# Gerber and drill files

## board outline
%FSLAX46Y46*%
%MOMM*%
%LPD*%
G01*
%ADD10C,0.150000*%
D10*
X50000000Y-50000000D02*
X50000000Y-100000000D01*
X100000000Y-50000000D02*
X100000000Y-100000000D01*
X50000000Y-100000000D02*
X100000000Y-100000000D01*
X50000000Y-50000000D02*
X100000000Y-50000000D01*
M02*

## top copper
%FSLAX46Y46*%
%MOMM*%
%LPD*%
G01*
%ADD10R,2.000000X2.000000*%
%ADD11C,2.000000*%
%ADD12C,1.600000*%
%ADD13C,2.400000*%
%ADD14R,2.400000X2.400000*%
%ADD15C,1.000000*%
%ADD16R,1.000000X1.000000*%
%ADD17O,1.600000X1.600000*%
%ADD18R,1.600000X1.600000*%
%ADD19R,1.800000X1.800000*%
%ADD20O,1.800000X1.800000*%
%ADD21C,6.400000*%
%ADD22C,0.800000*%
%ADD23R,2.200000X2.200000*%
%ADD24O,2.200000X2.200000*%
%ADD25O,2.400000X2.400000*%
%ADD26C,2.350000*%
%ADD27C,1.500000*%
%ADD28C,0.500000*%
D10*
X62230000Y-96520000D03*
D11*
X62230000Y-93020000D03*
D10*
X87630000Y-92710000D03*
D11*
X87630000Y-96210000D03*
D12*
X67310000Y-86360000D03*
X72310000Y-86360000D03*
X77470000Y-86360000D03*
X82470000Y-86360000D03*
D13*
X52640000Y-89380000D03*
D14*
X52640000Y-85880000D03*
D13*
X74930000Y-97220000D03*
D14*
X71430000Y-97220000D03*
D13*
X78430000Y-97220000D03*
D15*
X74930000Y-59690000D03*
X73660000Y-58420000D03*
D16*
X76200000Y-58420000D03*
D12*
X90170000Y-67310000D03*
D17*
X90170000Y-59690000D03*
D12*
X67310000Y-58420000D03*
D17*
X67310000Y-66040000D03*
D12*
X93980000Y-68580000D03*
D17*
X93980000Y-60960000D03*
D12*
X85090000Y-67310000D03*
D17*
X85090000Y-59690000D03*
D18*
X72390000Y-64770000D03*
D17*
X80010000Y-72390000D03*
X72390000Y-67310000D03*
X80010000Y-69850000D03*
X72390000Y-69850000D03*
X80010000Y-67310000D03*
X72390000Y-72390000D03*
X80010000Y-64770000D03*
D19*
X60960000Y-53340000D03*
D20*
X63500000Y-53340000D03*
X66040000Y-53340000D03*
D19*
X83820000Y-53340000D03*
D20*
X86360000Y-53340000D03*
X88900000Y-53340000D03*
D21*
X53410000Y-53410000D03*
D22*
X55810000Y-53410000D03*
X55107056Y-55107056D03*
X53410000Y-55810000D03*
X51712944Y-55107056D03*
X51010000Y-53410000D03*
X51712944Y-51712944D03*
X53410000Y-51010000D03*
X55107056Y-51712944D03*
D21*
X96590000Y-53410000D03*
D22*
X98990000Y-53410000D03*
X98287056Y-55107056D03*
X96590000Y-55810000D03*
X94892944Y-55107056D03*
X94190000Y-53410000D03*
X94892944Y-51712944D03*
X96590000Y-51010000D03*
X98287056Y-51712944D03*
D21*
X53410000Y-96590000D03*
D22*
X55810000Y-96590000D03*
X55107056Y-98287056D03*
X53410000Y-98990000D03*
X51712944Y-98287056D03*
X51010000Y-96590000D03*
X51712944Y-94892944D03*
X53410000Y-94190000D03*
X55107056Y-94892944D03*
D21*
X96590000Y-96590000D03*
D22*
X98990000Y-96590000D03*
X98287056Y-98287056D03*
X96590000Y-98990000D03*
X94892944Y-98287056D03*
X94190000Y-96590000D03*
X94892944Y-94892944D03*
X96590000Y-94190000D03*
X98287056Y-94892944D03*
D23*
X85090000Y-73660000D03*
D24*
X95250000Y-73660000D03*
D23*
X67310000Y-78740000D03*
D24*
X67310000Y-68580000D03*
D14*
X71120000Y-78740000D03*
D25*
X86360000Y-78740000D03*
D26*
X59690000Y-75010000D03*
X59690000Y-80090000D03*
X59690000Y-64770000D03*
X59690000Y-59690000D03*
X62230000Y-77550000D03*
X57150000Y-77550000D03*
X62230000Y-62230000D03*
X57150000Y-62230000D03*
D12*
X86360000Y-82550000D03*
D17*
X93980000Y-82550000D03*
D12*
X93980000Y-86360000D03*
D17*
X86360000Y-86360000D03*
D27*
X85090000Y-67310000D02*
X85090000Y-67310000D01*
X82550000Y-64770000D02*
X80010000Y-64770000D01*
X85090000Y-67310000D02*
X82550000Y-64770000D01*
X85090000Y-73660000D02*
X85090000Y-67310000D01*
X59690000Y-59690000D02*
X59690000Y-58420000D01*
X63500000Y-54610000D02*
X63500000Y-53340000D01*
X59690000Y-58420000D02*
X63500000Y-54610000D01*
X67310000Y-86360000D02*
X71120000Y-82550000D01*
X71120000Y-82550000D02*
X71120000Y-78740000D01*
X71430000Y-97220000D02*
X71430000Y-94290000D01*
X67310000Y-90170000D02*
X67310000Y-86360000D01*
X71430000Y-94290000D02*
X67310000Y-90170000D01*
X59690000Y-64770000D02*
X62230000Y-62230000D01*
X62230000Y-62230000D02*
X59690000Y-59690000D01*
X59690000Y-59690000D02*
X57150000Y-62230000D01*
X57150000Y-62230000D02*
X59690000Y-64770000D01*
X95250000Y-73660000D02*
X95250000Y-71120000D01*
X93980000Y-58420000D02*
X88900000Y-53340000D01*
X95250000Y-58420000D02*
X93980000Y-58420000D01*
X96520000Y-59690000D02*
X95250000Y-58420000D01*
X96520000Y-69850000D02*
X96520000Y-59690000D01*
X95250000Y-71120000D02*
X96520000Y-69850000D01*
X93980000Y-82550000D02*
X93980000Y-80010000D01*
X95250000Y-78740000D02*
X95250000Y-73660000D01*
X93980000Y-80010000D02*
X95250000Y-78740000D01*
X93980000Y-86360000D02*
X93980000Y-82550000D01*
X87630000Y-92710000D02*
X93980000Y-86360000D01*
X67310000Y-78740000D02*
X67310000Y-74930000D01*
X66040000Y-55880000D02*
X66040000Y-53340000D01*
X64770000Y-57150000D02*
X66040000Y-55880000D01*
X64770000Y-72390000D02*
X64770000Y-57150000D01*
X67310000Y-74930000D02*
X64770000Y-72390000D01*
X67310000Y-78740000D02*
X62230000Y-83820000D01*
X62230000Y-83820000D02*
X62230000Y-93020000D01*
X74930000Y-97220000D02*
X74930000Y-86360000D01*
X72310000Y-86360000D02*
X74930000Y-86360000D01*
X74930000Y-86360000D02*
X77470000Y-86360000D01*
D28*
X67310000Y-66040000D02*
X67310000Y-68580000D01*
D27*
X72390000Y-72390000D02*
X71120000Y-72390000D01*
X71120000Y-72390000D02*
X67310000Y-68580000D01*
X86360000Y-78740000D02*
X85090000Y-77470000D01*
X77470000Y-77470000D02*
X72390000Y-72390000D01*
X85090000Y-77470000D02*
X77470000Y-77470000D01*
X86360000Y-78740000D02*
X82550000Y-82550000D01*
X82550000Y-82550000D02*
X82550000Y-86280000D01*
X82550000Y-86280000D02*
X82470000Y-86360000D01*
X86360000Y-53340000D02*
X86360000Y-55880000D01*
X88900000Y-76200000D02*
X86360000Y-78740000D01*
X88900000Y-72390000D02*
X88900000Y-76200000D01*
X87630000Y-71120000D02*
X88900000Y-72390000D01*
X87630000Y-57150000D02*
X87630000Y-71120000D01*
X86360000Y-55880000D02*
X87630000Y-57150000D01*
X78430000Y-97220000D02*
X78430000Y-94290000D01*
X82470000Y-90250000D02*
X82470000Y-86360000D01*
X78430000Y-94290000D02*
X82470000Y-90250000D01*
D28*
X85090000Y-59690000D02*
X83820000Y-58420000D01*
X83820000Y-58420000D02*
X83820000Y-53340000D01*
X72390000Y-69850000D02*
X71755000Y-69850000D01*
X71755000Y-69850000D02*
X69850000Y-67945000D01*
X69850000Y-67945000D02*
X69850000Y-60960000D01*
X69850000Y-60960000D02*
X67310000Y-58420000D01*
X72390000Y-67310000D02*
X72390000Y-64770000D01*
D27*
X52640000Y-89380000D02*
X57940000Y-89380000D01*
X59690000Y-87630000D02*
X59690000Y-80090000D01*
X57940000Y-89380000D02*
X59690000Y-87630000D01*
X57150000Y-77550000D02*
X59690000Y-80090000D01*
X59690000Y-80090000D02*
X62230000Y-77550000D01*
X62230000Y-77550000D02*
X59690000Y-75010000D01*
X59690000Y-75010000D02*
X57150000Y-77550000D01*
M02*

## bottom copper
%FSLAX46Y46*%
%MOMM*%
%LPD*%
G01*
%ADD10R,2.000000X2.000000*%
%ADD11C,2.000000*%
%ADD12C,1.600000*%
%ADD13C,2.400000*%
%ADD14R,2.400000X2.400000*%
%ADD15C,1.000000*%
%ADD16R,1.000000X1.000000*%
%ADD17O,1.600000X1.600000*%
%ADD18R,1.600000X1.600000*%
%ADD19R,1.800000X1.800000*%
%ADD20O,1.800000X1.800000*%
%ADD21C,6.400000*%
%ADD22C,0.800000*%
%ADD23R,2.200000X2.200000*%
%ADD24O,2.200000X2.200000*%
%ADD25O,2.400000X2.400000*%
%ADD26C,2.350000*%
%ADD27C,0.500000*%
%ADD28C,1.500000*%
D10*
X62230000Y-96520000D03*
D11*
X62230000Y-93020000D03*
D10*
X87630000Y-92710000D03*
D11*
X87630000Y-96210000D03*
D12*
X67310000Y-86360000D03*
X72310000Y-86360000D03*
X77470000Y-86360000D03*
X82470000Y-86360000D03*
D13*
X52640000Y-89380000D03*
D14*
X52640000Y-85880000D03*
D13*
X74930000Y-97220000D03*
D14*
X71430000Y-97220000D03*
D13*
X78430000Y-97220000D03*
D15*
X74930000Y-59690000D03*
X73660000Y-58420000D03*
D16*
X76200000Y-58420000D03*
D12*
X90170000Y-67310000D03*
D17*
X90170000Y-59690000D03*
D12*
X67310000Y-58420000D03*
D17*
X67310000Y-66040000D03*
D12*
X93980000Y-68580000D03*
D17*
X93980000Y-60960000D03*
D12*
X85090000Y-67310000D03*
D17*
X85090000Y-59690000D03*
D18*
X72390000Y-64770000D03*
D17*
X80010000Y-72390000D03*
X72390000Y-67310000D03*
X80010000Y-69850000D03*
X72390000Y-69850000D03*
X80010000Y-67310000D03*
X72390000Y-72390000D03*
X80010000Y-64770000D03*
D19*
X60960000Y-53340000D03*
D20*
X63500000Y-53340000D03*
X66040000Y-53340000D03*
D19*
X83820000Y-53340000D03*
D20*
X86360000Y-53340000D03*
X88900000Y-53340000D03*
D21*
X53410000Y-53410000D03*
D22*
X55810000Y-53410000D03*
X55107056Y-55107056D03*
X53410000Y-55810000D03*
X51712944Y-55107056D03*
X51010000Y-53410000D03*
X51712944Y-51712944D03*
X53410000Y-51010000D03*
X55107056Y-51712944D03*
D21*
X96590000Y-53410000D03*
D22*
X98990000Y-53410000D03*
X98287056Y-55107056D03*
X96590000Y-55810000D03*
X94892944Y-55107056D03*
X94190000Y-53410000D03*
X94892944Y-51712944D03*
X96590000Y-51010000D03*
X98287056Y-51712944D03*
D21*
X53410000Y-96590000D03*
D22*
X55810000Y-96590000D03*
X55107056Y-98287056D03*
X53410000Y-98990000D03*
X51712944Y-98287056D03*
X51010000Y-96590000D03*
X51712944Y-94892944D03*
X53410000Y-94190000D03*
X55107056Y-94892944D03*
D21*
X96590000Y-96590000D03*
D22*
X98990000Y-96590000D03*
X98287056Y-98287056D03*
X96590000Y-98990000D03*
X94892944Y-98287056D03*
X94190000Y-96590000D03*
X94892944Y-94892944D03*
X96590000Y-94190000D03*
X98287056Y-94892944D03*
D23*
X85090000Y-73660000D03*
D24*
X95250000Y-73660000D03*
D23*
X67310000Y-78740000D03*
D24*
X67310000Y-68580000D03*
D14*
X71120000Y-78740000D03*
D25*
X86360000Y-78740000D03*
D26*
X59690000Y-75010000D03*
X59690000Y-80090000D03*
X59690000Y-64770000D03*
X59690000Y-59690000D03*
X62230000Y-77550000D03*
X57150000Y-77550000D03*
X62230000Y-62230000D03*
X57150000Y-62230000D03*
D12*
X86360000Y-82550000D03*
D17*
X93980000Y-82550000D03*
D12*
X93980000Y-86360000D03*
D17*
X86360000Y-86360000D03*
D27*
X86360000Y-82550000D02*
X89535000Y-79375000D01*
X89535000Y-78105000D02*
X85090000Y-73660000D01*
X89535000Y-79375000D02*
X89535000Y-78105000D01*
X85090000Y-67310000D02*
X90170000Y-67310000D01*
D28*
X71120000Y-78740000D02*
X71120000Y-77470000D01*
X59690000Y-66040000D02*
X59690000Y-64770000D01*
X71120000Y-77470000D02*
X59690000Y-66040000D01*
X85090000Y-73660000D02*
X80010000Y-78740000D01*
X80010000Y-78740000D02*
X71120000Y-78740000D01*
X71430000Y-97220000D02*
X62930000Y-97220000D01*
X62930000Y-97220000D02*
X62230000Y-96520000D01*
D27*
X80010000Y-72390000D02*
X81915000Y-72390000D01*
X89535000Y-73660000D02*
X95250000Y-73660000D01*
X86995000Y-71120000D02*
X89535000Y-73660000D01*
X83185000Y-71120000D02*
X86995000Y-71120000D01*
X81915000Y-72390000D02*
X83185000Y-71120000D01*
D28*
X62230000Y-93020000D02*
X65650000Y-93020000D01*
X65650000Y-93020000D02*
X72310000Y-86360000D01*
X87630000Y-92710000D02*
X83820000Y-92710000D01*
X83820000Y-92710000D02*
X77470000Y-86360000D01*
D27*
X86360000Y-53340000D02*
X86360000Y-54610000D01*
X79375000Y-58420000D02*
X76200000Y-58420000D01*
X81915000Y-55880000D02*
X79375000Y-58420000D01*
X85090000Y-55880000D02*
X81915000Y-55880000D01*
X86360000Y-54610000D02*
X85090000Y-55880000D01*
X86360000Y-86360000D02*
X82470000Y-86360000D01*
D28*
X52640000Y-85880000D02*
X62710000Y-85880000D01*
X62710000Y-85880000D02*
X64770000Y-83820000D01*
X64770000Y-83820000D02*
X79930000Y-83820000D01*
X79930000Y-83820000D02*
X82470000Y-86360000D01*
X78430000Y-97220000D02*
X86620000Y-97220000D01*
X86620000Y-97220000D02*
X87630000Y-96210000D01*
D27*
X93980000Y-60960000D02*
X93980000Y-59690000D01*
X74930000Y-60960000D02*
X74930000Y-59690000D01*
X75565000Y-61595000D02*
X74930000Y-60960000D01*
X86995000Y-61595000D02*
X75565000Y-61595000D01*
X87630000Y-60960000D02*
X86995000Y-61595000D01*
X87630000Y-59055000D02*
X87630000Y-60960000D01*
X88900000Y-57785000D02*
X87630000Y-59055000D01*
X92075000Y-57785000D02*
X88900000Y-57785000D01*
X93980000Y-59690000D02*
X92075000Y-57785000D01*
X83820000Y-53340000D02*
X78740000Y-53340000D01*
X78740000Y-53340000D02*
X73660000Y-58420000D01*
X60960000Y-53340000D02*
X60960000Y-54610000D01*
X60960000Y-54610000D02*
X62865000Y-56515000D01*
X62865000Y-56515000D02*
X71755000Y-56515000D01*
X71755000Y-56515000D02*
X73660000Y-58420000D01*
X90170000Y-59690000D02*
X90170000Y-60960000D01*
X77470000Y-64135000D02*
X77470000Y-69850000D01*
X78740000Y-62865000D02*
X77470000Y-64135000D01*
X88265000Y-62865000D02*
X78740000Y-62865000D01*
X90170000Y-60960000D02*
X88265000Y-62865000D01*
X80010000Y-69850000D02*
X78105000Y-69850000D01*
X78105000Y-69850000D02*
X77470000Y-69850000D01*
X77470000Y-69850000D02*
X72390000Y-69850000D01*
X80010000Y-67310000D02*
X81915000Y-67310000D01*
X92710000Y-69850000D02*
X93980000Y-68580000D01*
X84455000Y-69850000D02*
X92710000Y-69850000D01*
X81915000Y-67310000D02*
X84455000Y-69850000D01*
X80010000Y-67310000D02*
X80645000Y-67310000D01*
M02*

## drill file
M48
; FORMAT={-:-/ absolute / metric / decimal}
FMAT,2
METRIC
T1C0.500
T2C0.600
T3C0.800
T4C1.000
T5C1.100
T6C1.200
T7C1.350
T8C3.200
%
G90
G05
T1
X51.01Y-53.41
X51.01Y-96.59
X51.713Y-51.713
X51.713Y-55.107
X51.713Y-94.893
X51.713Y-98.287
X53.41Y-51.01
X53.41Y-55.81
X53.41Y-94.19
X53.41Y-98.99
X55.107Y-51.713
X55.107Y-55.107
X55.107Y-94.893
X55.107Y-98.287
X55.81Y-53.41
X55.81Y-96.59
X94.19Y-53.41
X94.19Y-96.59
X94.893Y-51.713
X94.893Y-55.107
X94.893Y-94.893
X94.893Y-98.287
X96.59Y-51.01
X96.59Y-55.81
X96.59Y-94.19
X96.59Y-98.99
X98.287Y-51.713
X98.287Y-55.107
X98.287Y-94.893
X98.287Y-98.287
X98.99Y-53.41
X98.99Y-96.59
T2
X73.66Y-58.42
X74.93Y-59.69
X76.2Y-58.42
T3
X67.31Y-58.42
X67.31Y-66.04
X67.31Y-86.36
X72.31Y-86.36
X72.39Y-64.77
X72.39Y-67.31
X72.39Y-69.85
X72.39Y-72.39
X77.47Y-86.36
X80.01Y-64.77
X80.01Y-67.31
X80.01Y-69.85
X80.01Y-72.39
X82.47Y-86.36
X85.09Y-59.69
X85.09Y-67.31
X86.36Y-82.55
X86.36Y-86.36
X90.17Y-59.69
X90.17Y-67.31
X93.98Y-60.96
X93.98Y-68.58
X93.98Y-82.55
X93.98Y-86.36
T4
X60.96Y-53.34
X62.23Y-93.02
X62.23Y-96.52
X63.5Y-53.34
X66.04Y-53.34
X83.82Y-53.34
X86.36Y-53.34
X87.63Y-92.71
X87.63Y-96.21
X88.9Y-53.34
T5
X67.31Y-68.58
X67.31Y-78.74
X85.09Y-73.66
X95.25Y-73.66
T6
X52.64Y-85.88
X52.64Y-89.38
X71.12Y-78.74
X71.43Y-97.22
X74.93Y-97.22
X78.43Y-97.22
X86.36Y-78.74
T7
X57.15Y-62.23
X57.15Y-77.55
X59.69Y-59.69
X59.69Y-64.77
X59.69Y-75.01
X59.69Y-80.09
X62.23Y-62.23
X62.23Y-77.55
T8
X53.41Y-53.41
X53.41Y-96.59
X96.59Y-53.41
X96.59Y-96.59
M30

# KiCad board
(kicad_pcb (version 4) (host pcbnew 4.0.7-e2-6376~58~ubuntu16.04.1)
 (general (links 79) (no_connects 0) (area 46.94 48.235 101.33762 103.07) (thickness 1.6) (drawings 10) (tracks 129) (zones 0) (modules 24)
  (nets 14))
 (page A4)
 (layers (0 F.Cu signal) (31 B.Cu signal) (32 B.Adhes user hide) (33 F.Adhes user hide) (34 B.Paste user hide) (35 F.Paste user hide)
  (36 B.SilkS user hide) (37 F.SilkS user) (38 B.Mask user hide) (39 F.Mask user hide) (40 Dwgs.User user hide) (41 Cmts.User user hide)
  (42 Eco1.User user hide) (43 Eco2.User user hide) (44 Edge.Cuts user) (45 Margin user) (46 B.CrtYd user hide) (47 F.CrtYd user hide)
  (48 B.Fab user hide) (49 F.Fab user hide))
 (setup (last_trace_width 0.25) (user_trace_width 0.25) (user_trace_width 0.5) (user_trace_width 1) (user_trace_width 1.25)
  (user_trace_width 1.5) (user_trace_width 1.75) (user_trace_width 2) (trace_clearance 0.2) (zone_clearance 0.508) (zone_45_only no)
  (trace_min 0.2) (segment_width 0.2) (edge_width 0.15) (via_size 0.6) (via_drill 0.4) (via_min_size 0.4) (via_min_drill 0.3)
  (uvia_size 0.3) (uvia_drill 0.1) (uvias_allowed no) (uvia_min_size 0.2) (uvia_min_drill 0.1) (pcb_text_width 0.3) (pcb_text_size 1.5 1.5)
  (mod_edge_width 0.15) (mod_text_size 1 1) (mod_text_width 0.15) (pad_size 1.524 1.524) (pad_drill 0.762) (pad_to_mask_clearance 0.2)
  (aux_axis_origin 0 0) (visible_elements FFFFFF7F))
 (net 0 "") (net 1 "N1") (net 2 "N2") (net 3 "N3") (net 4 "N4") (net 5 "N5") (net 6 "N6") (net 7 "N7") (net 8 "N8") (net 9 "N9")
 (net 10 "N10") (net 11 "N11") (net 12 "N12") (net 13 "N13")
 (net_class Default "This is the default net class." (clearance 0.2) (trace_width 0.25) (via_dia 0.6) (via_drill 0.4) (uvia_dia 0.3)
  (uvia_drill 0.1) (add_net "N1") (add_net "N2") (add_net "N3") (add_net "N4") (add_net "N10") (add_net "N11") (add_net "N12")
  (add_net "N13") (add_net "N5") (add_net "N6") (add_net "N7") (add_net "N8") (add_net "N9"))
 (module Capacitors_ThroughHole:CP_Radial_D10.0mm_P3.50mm (layer F.Cu) (at 62.23 96.52 90)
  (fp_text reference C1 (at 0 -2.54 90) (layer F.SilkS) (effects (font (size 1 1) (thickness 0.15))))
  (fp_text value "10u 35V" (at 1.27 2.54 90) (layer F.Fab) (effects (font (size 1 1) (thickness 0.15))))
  (pad 1 thru_hole rect (at 0 0 90) (size 2 2) (drill 1) (layers *.Cu *.Mask) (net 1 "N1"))
  (pad 2 thru_hole circle (at 3.5 0 90) (size 2 2) (drill 1) (layers *.Cu *.Mask) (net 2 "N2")))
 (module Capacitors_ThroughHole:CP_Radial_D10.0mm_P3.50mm (layer F.Cu) (at 87.63 92.71 270)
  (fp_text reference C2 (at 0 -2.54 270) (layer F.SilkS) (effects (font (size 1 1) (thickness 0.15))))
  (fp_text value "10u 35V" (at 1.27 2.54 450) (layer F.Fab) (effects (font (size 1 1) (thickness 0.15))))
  (pad 1 thru_hole rect (at 0 0 270) (size 2 2) (drill 1) (layers *.Cu *.Mask) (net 2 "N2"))
  (pad 2 thru_hole circle (at 3.5 0 270) (size 2 2) (drill 1) (layers *.Cu *.Mask) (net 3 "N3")))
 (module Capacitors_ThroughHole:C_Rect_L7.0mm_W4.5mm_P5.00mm (layer F.Cu) (at 67.31 86.36)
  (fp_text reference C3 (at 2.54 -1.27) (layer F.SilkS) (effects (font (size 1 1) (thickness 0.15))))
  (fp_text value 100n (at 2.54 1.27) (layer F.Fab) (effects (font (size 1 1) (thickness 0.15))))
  (pad 1 thru_hole circle (at 0 0) (size 1.6 1.6) (drill 0.8) (layers *.Cu *.Mask) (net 1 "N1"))
  (pad 2 thru_hole circle (at 5 0) (size 1.6 1.6) (drill 0.8) (layers *.Cu *.Mask) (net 2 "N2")))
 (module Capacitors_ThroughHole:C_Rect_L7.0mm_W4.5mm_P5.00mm (layer F.Cu) (at 77.47 86.36)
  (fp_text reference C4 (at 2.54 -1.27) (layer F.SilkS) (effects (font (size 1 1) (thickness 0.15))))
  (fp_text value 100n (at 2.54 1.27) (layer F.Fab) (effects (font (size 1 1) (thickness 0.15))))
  (pad 1 thru_hole circle (at 0 0) (size 1.6 1.6) (drill 0.8) (layers *.Cu *.Mask) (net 2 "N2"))
  (pad 2 thru_hole circle (at 5 0) (size 1.6 1.6) (drill 0.8) (layers *.Cu *.Mask) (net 3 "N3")))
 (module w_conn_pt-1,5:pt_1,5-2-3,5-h (layer F.Cu) (at 53.34 87.63 90)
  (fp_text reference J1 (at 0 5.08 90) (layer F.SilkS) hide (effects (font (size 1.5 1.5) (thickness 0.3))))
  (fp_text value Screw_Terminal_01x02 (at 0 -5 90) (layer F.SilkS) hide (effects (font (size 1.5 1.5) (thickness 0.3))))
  (pad 2 thru_hole circle (at -1.75 -0.7 90) (size 2.4 2.4) (drill 1.2) (layers *.Cu *.Mask F.SilkS) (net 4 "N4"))
  (pad 1 thru_hole rect (at 1.75 -0.7 90) (size 2.4 2.4) (drill 1.2) (layers *.Cu *.Mask F.SilkS) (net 3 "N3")))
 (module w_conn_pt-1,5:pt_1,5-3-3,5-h (layer F.Cu) (at 74.93 96.52 180)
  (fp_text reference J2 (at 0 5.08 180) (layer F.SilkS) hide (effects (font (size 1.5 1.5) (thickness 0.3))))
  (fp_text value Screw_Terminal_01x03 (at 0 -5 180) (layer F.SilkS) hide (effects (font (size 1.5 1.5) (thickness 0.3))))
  (pad 2 thru_hole circle (at 0 -0.7 180) (size 2.4 2.4) (drill 1.2) (layers *.Cu *.Mask F.SilkS) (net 2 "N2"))
  (pad 1 thru_hole rect (at 3.5 -0.7 180) (size 2.4 2.4) (drill 1.2) (layers *.Cu *.Mask F.SilkS) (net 1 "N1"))
  (pad 3 thru_hole circle (at -3.5 -0.7 180) (size 2.4 2.4) (drill 1.2) (layers *.Cu *.Mask F.SilkS) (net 3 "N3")))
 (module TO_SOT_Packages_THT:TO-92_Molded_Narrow (layer F.Cu) (at 76.2 58.42 180)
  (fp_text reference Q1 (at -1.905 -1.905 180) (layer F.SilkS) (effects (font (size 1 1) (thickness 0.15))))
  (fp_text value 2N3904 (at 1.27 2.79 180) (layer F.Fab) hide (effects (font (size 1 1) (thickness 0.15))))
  (pad 2 thru_hole circle (at 1.27 -1.27 270) (size 1 1) (drill 0.6) (layers *.Cu *.Mask) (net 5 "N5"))
  (pad 3 thru_hole circle (at 2.54 0 270) (size 1 1) (drill 0.6) (layers *.Cu *.Mask) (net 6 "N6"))
  (pad 1 thru_hole rect (at 0 0 270) (size 1 1) (drill 0.6) (layers *.Cu *.Mask) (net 3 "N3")))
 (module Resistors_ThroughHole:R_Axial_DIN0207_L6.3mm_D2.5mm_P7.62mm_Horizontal (layer F.Cu) (at 90.17 67.31 90)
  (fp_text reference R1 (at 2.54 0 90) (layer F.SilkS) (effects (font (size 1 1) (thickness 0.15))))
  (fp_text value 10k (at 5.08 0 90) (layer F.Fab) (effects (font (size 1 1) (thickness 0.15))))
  (pad 1 thru_hole circle (at 0 0 90) (size 1.6 1.6) (drill 0.8) (layers *.Cu *.Mask) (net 1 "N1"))
  (pad 2 thru_hole oval (at 7.62 0 90) (size 1.6 1.6) (drill 0.8) (layers *.Cu *.Mask) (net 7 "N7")))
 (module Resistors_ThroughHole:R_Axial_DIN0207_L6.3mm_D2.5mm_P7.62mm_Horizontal (layer F.Cu) (at 67.31 58.42 270)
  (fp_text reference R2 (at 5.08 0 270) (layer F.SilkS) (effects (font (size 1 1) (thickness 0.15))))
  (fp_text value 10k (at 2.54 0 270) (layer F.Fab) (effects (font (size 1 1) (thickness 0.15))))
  (pad 1 thru_hole circle (at 0 0 270) (size 1.6 1.6) (drill 0.8) (layers *.Cu *.Mask) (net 7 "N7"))
  (pad 2 thru_hole oval (at 7.62 0 270) (size 1.6 1.6) (drill 0.8) (layers *.Cu *.Mask) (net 3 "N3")))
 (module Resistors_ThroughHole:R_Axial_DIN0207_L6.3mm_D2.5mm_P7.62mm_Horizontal (layer F.Cu) (at 93.98 68.58 90)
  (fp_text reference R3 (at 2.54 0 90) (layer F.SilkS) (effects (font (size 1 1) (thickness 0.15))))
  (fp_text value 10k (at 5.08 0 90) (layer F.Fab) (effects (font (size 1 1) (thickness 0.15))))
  (pad 1 thru_hole circle (at 0 0 90) (size 1.6 1.6) (drill 0.8) (layers *.Cu *.Mask) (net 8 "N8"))
  (pad 2 thru_hole oval (at 7.62 0 90) (size 1.6 1.6) (drill 0.8) (layers *.Cu *.Mask) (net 5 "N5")))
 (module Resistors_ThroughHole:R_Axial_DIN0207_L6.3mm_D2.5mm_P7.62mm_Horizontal (layer F.Cu) (at 85.09 67.31 90)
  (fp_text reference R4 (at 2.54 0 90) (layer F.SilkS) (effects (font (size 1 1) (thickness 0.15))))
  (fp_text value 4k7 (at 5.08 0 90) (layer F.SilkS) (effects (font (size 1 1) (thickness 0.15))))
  (pad 1 thru_hole circle (at 0 0 90) (size 1.6 1.6) (drill 0.8) (layers *.Cu *.Mask) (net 1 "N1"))
  (pad 2 thru_hole oval (at 7.62 0 90) (size 1.6 1.6) (drill 0.8) (layers *.Cu *.Mask) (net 6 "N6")))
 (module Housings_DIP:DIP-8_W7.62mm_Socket (layer F.Cu) (at 72.39 64.77)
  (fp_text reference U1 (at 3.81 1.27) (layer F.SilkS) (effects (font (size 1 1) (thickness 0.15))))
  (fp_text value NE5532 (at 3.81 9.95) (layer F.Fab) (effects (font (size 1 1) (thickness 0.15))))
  (pad 1 thru_hole rect (at 0 0) (size 1.6 1.6) (drill 0.8) (layers *.Cu *.Mask) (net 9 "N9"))
  (pad 5 thru_hole oval (at 7.62 7.62) (size 1.6 1.6) (drill 0.8) (layers *.Cu *.Mask) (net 2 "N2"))
  (pad 2 thru_hole oval (at 0 2.54) (size 1.6 1.6) (drill 0.8) (layers *.Cu *.Mask) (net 9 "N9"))
  (pad 6 thru_hole oval (at 7.62 5.08) (size 1.6 1.6) (drill 0.8) (layers *.Cu *.Mask) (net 7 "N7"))
  (pad 3 thru_hole oval (at 0 5.08) (size 1.6 1.6) (drill 0.8) (layers *.Cu *.Mask) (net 7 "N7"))
  (pad 7 thru_hole oval (at 7.62 2.54) (size 1.6 1.6) (drill 0.8) (layers *.Cu *.Mask) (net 8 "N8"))
  (pad 4 thru_hole oval (at 0 7.62) (size 1.6 1.6) (drill 0.8) (layers *.Cu *.Mask) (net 3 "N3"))
  (pad 8 thru_hole oval (at 7.62 0) (size 1.6 1.6) (drill 0.8) (layers *.Cu *.Mask) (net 1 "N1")))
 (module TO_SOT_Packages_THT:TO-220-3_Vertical (layer F.Cu) (at 60.96 53.34)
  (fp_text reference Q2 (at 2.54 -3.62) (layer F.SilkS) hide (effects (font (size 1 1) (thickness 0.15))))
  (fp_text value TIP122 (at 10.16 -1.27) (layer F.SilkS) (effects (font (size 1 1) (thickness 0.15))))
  (pad 1 thru_hole rect (at 0 0) (size 1.8 1.8) (drill 1) (layers *.Cu *.Mask) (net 6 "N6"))
  (pad 2 thru_hole oval (at 2.54 0) (size 1.8 1.8) (drill 1) (layers *.Cu *.Mask) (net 1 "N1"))
  (pad 3 thru_hole oval (at 5.08 0) (size 1.8 1.8) (drill 1) (layers *.Cu *.Mask) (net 2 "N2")))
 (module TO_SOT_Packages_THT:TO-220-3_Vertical (layer F.Cu) (at 83.82 53.34)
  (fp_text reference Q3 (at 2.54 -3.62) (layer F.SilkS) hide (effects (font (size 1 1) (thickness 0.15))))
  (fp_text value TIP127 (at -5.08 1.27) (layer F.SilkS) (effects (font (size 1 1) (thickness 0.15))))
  (pad 1 thru_hole rect (at 0 0) (size 1.8 1.8) (drill 1) (layers *.Cu *.Mask) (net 6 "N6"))
  (pad 2 thru_hole oval (at 2.54 0) (size 1.8 1.8) (drill 1) (layers *.Cu *.Mask) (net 3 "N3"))
  (pad 3 thru_hole oval (at 5.08 0) (size 1.8 1.8) (drill 1) (layers *.Cu *.Mask) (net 2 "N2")))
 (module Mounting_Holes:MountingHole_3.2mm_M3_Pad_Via (layer F.Cu) (at 53.41 53.41)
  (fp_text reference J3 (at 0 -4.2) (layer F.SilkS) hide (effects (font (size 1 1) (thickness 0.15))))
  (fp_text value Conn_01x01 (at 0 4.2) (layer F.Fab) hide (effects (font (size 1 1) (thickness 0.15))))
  (pad 1 thru_hole circle (at 0 0) (size 6.4 6.4) (drill 3.2) (layers *.Cu *.Mask) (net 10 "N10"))
  (pad 1 thru_hole circle (at 2.4 0) (size 0.8 0.8) (drill 0.5) (layers *.Cu *.Mask) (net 10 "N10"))
  (pad 1 thru_hole circle (at 1.697056 1.697056) (size 0.8 0.8) (drill 0.5) (layers *.Cu *.Mask) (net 10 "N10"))
  (pad 1 thru_hole circle (at 0 2.4) (size 0.8 0.8) (drill 0.5) (layers *.Cu *.Mask) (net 10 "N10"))
  (pad 1 thru_hole circle (at -1.697056 1.697056) (size 0.8 0.8) (drill 0.5) (layers *.Cu *.Mask) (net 10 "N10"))
  (pad 1 thru_hole circle (at -2.4 0) (size 0.8 0.8) (drill 0.5) (layers *.Cu *.Mask) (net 10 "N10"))
  (pad 1 thru_hole circle (at -1.697056 -1.697056) (size 0.8 0.8) (drill 0.5) (layers *.Cu *.Mask) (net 10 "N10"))
  (pad 1 thru_hole circle (at 0 -2.4) (size 0.8 0.8) (drill 0.5) (layers *.Cu *.Mask) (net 10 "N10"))
  (pad 1 thru_hole circle (at 1.697056 -1.697056) (size 0.8 0.8) (drill 0.5) (layers *.Cu *.Mask) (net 10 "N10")))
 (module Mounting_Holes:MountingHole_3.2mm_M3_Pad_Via (layer F.Cu) (at 96.59 53.41)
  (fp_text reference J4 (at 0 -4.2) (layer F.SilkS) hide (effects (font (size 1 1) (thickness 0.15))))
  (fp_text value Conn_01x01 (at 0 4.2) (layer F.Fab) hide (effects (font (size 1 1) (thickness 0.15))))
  (pad 1 thru_hole circle (at 0 0) (size 6.4 6.4) (drill 3.2) (layers *.Cu *.Mask) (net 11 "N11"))
  (pad 1 thru_hole circle (at 2.4 0) (size 0.8 0.8) (drill 0.5) (layers *.Cu *.Mask) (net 11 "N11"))
  (pad 1 thru_hole circle (at 1.697056 1.697056) (size 0.8 0.8) (drill 0.5) (layers *.Cu *.Mask) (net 11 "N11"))
  (pad 1 thru_hole circle (at 0 2.4) (size 0.8 0.8) (drill 0.5) (layers *.Cu *.Mask) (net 11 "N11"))
  (pad 1 thru_hole circle (at -1.697056 1.697056) (size 0.8 0.8) (drill 0.5) (layers *.Cu *.Mask) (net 11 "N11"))
  (pad 1 thru_hole circle (at -2.4 0) (size 0.8 0.8) (drill 0.5) (layers *.Cu *.Mask) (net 11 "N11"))
  (pad 1 thru_hole circle (at -1.697056 -1.697056) (size 0.8 0.8) (drill 0.5) (layers *.Cu *.Mask) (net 11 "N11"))
  (pad 1 thru_hole circle (at 0 -2.4) (size 0.8 0.8) (drill 0.5) (layers *.Cu *.Mask) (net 11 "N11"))
  (pad 1 thru_hole circle (at 1.697056 -1.697056) (size 0.8 0.8) (drill 0.5) (layers *.Cu *.Mask) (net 11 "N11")))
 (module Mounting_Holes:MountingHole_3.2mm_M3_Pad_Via (layer F.Cu) (at 53.41 96.59)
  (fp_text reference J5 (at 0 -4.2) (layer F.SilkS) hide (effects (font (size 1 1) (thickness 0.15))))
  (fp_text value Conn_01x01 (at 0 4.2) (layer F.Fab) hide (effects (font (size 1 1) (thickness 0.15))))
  (pad 1 thru_hole circle (at 0 0) (size 6.4 6.4) (drill 3.2) (layers *.Cu *.Mask) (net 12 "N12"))
  (pad 1 thru_hole circle (at 2.4 0) (size 0.8 0.8) (drill 0.5) (layers *.Cu *.Mask) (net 12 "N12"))
  (pad 1 thru_hole circle (at 1.697056 1.697056) (size 0.8 0.8) (drill 0.5) (layers *.Cu *.Mask) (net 12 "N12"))
  (pad 1 thru_hole circle (at 0 2.4) (size 0.8 0.8) (drill 0.5) (layers *.Cu *.Mask) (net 12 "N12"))
  (pad 1 thru_hole circle (at -1.697056 1.697056) (size 0.8 0.8) (drill 0.5) (layers *.Cu *.Mask) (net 12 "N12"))
  (pad 1 thru_hole circle (at -2.4 0) (size 0.8 0.8) (drill 0.5) (layers *.Cu *.Mask) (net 12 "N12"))
  (pad 1 thru_hole circle (at -1.697056 -1.697056) (size 0.8 0.8) (drill 0.5) (layers *.Cu *.Mask) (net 12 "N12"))
  (pad 1 thru_hole circle (at 0 -2.4) (size 0.8 0.8) (drill 0.5) (layers *.Cu *.Mask) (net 12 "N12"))
  (pad 1 thru_hole circle (at 1.697056 -1.697056) (size 0.8 0.8) (drill 0.5) (layers *.Cu *.Mask) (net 12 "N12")))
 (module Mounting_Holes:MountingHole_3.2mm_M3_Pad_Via (layer F.Cu) (at 96.59 96.59)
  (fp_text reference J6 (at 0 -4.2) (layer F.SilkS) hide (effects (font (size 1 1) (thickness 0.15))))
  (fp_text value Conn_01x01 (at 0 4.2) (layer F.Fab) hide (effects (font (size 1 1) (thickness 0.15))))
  (pad 1 thru_hole circle (at 0 0) (size 6.4 6.4) (drill 3.2) (layers *.Cu *.Mask) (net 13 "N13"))
  (pad 1 thru_hole circle (at 2.4 0) (size 0.8 0.8) (drill 0.5) (layers *.Cu *.Mask) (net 13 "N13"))
  (pad 1 thru_hole circle (at 1.697056 1.697056) (size 0.8 0.8) (drill 0.5) (layers *.Cu *.Mask) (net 13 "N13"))
  (pad 1 thru_hole circle (at 0 2.4) (size 0.8 0.8) (drill 0.5) (layers *.Cu *.Mask) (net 13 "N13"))
  (pad 1 thru_hole circle (at -1.697056 1.697056) (size 0.8 0.8) (drill 0.5) (layers *.Cu *.Mask) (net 13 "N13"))
  (pad 1 thru_hole circle (at -2.4 0) (size 0.8 0.8) (drill 0.5) (layers *.Cu *.Mask) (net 13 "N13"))
  (pad 1 thru_hole circle (at -1.697056 -1.697056) (size 0.8 0.8) (drill 0.5) (layers *.Cu *.Mask) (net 13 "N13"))
  (pad 1 thru_hole circle (at 0 -2.4) (size 0.8 0.8) (drill 0.5) (layers *.Cu *.Mask) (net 13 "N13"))
  (pad 1 thru_hole circle (at 1.697056 -1.697056) (size 0.8 0.8) (drill 0.5) (layers *.Cu *.Mask) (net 13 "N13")))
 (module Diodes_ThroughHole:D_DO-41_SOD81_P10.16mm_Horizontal (layer F.Cu) (at 85.09 73.66)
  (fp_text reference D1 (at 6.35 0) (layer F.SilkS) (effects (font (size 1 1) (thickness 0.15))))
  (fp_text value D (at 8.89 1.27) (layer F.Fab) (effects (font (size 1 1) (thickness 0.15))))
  (pad 1 thru_hole rect (at 0 0) (size 2.2 2.2) (drill 1.1) (layers *.Cu *.Mask) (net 1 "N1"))
  (pad 2 thru_hole oval (at 10.16 0) (size 2.2 2.2) (drill 1.1) (layers *.Cu *.Mask) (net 2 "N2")))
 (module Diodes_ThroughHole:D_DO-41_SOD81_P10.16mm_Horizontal (layer F.Cu) (at 67.31 78.74 90)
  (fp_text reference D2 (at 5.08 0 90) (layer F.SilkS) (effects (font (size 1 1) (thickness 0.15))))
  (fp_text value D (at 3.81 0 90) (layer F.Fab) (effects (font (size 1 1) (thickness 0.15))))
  (pad 1 thru_hole rect (at 0 0 90) (size 2.2 2.2) (drill 1.1) (layers *.Cu *.Mask) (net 2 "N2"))
  (pad 2 thru_hole oval (at 10.16 0 90) (size 2.2 2.2) (drill 1.1) (layers *.Cu *.Mask) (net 3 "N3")))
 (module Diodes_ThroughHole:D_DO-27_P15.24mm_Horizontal (layer F.Cu) (at 71.12 78.74)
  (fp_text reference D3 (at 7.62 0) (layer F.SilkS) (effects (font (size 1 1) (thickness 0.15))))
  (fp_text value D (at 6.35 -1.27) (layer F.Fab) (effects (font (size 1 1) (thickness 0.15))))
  (pad 1 thru_hole rect (at 0 0) (size 2.4 2.4) (drill 1.2) (layers *.Cu *.Mask) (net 1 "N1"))
  (pad 2 thru_hole oval (at 15.24 0) (size 2.4 2.4) (drill 1.2) (layers *.Cu *.Mask) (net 3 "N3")))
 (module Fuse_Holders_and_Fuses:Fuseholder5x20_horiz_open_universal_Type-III (layer F.Cu) (at 59.69 59.69 270)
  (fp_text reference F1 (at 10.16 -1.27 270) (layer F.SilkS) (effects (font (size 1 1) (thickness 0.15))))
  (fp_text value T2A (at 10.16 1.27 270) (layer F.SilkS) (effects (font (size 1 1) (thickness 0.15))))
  (pad 2 thru_hole circle (at 15.32 0 270) (size 2.35 2.35) (drill 1.35) (layers *.Cu *.Mask) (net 4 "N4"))
  (pad 2 thru_hole circle (at 20.4 0 270) (size 2.35 2.35) (drill 1.35) (layers *.Cu *.Mask) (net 4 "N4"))
  (pad 1 thru_hole circle (at 5.08 0 270) (size 2.35 2.35) (drill 1.35) (layers *.Cu *.Mask) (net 1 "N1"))
  (pad 1 thru_hole circle (at 0 0 270) (size 2.35 2.35) (drill 1.35) (layers *.Cu *.Mask) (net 1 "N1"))
  (pad 2 thru_hole circle (at 17.86 -2.54 270) (size 2.35 2.35) (drill 1.35) (layers *.Cu *.Mask) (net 4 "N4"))
  (pad 2 thru_hole circle (at 17.86 2.54 270) (size 2.35 2.35) (drill 1.35) (layers *.Cu *.Mask) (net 4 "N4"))
  (pad 1 thru_hole circle (at 2.54 -2.54 270) (size 2.35 2.35) (drill 1.35) (layers *.Cu *.Mask) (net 1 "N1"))
  (pad 1 thru_hole circle (at 2.54 2.54 270) (size 2.35 2.35) (drill 1.35) (layers *.Cu *.Mask) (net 1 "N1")))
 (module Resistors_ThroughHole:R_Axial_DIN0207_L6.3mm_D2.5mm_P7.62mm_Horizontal (layer F.Cu) (at 86.36 82.55)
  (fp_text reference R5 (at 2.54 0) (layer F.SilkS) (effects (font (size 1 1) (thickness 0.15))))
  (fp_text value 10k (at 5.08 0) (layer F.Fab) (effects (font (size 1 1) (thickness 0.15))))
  (pad 1 thru_hole circle (at 0 0) (size 1.6 1.6) (drill 0.8) (layers *.Cu *.Mask) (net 1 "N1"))
  (pad 2 thru_hole oval (at 7.62 0) (size 1.6 1.6) (drill 0.8) (layers *.Cu *.Mask) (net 2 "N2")))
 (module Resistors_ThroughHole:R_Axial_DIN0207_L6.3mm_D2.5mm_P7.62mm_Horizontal (layer F.Cu) (at 93.98 86.36 180)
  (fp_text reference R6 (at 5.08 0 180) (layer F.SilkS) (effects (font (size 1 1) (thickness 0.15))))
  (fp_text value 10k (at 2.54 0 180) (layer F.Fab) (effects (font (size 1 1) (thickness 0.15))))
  (pad 1 thru_hole circle (at 0 0 180) (size 1.6 1.6) (drill 0.8) (layers *.Cu *.Mask) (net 2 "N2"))
  (pad 2 thru_hole oval (at 7.62 0 180) (size 1.6 1.6) (drill 0.8) (layers *.Cu *.Mask) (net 3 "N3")))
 (gr_line (start 50 50) (end 50 100) (angle 90) (layer Edge.Cuts) (width 0.15))
 (gr_line (start 100 50) (end 100 100) (angle 90) (layer Edge.Cuts) (width 0.15))
 (gr_line (start 50 100) (end 100 100) (angle 90) (layer Edge.Cuts) (width 0.15))
 (gr_line (start 50 50) (end 100 50) (angle 90) (layer Edge.Cuts) (width 0.15))
 (segment (start 86.36 82.55) (end 89.535 79.375) (width 0.5) (layer B.Cu) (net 1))
 (segment (start 89.535 78.105) (end 85.09 73.66) (width 0.5) (layer B.Cu) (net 1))
 (segment (start 89.535 79.375) (end 89.535 78.105) (width 0.5) (layer B.Cu) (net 1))
 (segment (start 85.09 67.31) (end 90.17 67.31) (width 0.5) (layer B.Cu) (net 1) (status 20))
 (segment (start 85.09 67.31) (end 85.09 67.31) (width 1.5) (layer F.Cu) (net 1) (status 10))
 (segment (start 82.55 64.77) (end 80.01 64.77) (width 1.5) (layer F.Cu) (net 1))
 (segment (start 85.09 67.31) (end 82.55 64.77) (width 1.5) (layer F.Cu) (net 1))
 (segment (start 85.09 73.66) (end 85.09 67.31) (width 1.5) (layer F.Cu) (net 1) (status 20))
 (segment (start 59.69 59.69) (end 59.69 58.42) (width 1.5) (layer F.Cu) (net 1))
 (segment (start 63.5 54.61) (end 63.5 53.34) (width 1.5) (layer F.Cu) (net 1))
 (segment (start 59.69 58.42) (end 63.5 54.61) (width 1.5) (layer F.Cu) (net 1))
 (segment (start 71.12 78.74) (end 71.12 77.47) (width 1.5) (layer B.Cu) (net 1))
 (segment (start 59.69 66.04) (end 59.69 64.77) (width 1.5) (layer B.Cu) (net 1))
 (segment (start 71.12 77.47) (end 59.69 66.04) (width 1.5) (layer B.Cu) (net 1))
 (segment (start 85.09 73.66) (end 80.01 78.74) (width 1.5) (layer B.Cu) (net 1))
 (segment (start 80.01 78.74) (end 71.12 78.74) (width 1.5) (layer B.Cu) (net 1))
 (segment (start 67.31 86.36) (end 71.12 82.55) (width 1.5) (layer F.Cu) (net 1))
 (segment (start 71.12 82.55) (end 71.12 78.74) (width 1.5) (layer F.Cu) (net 1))
 (segment (start 71.43 97.22) (end 62.93 97.22) (width 1.5) (layer B.Cu) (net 1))
 (segment (start 62.93 97.22) (end 62.23 96.52) (width 1.5) (layer B.Cu) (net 1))
 (segment (start 71.43 97.22) (end 71.43 94.29) (width 1.5) (layer F.Cu) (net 1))
 (segment (start 67.31 90.17) (end 67.31 86.36) (width 1.5) (layer F.Cu) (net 1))
 (segment (start 71.43 94.29) (end 67.31 90.17) (width 1.5) (layer F.Cu) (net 1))
 (segment (start 59.69 64.77) (end 62.23 62.23) (width 1.5) (layer F.Cu) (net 1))
 (segment (start 62.23 62.23) (end 59.69 59.69) (width 1.5) (layer F.Cu) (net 1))
 (segment (start 59.69 59.69) (end 57.15 62.23) (width 1.5) (layer F.Cu) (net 1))
 (segment (start 57.15 62.23) (end 59.69 64.77) (width 1.5) (layer F.Cu) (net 1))
 (segment (start 80.01 72.39) (end 81.915 72.39) (width 0.5) (layer B.Cu) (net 2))
 (segment (start 89.535 73.66) (end 95.25 73.66) (width 0.5) (layer B.Cu) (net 2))
 (segment (start 86.995 71.12) (end 89.535 73.66) (width 0.5) (layer B.Cu) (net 2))
 (segment (start 83.185 71.12) (end 86.995 71.12) (width 0.5) (layer B.Cu) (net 2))
 (segment (start 81.915 72.39) (end 83.185 71.12) (width 0.5) (layer B.Cu) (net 2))
 (segment (start 95.25 73.66) (end 95.25 71.12) (width 1.5) (layer F.Cu) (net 2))
 (segment (start 93.98 58.42) (end 88.9 53.34) (width 1.5) (layer F.Cu) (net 2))
 (segment (start 95.25 58.42) (end 93.98 58.42) (width 1.5) (layer F.Cu) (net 2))
 (segment (start 96.52 59.69) (end 95.25 58.42) (width 1.5) (layer F.Cu) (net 2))
 (segment (start 96.52 69.85) (end 96.52 59.69) (width 1.5) (layer F.Cu) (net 2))
 (segment (start 95.25 71.12) (end 96.52 69.85) (width 1.5) (layer F.Cu) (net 2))
 (segment (start 93.98 82.55) (end 93.98 80.01) (width 1.5) (layer F.Cu) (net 2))
 (segment (start 95.25 78.74) (end 95.25 73.66) (width 1.5) (layer F.Cu) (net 2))
 (segment (start 93.98 80.01) (end 95.25 78.74) (width 1.5) (layer F.Cu) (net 2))
 (segment (start 93.98 86.36) (end 93.98 82.55) (width 1.5) (layer F.Cu) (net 2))
 (segment (start 87.63 92.71) (end 93.98 86.36) (width 1.5) (layer F.Cu) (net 2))
 (segment (start 67.31 78.74) (end 67.31 74.93) (width 1.5) (layer F.Cu) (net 2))
 (segment (start 66.04 55.88) (end 66.04 53.34) (width 1.5) (layer F.Cu) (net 2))
 (segment (start 64.77 57.15) (end 66.04 55.88) (width 1.5) (layer F.Cu) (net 2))
 (segment (start 64.77 72.39) (end 64.77 57.15) (width 1.5) (layer F.Cu) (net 2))
 (segment (start 67.31 74.93) (end 64.77 72.39) (width 1.5) (layer F.Cu) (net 2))
 (segment (start 67.31 78.74) (end 62.23 83.82) (width 1.5) (layer F.Cu) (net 2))
 (segment (start 62.23 83.82) (end 62.23 93.02) (width 1.5) (layer F.Cu) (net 2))
 (segment (start 62.23 93.02) (end 65.65 93.02) (width 1.5) (layer B.Cu) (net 2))
 (segment (start 65.65 93.02) (end 72.31 86.36) (width 1.5) (layer B.Cu) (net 2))
 (segment (start 87.63 92.71) (end 83.82 92.71) (width 1.5) (layer B.Cu) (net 2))
 (segment (start 83.82 92.71) (end 77.47 86.36) (width 1.5) (layer B.Cu) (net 2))
 (segment (start 74.93 97.22) (end 74.93 86.36) (width 1.5) (layer F.Cu) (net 2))
 (segment (start 72.31 86.36) (end 74.93 86.36) (width 1.5) (layer F.Cu) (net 2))
 (segment (start 74.93 86.36) (end 77.47 86.36) (width 1.5) (layer F.Cu) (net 2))
 (segment (start 67.31 66.04) (end 67.31 68.58) (width 0.5) (layer F.Cu) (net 3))
 (segment (start 86.36 53.34) (end 86.36 54.61) (width 0.5) (layer B.Cu) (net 3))
 (segment (start 79.375 58.42) (end 76.2 58.42) (width 0.5) (layer B.Cu) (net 3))
 (segment (start 81.915 55.88) (end 79.375 58.42) (width 0.5) (layer B.Cu) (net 3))
 (segment (start 85.09 55.88) (end 81.915 55.88) (width 0.5) (layer B.Cu) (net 3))
 (segment (start 86.36 54.61) (end 85.09 55.88) (width 0.5) (layer B.Cu) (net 3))
 (segment (start 86.36 86.36) (end 82.47 86.36) (width 0.5) (layer B.Cu) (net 3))
 (segment (start 72.39 72.39) (end 71.12 72.39) (width 1.5) (layer F.Cu) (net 3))
 (segment (start 71.12 72.39) (end 67.31 68.58) (width 1.5) (layer F.Cu) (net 3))
 (segment (start 86.36 78.74) (end 85.09 77.47) (width 1.5) (layer F.Cu) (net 3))
 (segment (start 77.47 77.47) (end 72.39 72.39) (width 1.5) (layer F.Cu) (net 3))
 (segment (start 85.09 77.47) (end 77.47 77.47) (width 1.5) (layer F.Cu) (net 3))
 (segment (start 86.36 78.74) (end 82.55 82.55) (width 1.5) (layer F.Cu) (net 3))
 (segment (start 82.55 82.55) (end 82.55 86.28) (width 1.5) (layer F.Cu) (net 3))
 (segment (start 82.55 86.28) (end 82.47 86.36) (width 1.5) (layer F.Cu) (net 3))
 (segment (start 86.36 53.34) (end 86.36 55.88) (width 1.5) (layer F.Cu) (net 3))
 (segment (start 88.9 76.2) (end 86.36 78.74) (width 1.5) (layer F.Cu) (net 3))
 (segment (start 88.9 72.39) (end 88.9 76.2) (width 1.5) (layer F.Cu) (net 3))
 (segment (start 87.63 71.12) (end 88.9 72.39) (width 1.5) (layer F.Cu) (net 3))
 (segment (start 87.63 57.15) (end 87.63 71.12) (width 1.5) (layer F.Cu) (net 3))
 (segment (start 86.36 55.88) (end 87.63 57.15) (width 1.5) (layer F.Cu) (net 3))
 (segment (start 78.43 97.22) (end 78.43 94.29) (width 1.5) (layer F.Cu) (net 3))
 (segment (start 82.47 90.25) (end 82.47 86.36) (width 1.5) (layer F.Cu) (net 3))
 (segment (start 78.43 94.29) (end 82.47 90.25) (width 1.5) (layer F.Cu) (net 3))
 (segment (start 52.64 85.88) (end 62.71 85.88) (width 1.5) (layer B.Cu) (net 3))
 (segment (start 62.71 85.88) (end 64.77 83.82) (width 1.5) (layer B.Cu) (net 3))
 (segment (start 64.77 83.82) (end 79.93 83.82) (width 1.5) (layer B.Cu) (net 3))
 (segment (start 79.93 83.82) (end 82.47 86.36) (width 1.5) (layer B.Cu) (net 3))
 (segment (start 78.43 97.22) (end 86.62 97.22) (width 1.5) (layer B.Cu) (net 3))
 (segment (start 86.62 97.22) (end 87.63 96.21) (width 1.5) (layer B.Cu) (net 3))
 (segment (start 93.98 60.96) (end 93.98 59.69) (width 0.5) (layer B.Cu) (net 5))
 (segment (start 74.93 60.96) (end 74.93 59.69) (width 0.5) (layer B.Cu) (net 5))
 (segment (start 75.565 61.595) (end 74.93 60.96) (width 0.5) (layer B.Cu) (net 5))
 (segment (start 86.995 61.595) (end 75.565 61.595) (width 0.5) (layer B.Cu) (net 5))
 (segment (start 87.63 60.96) (end 86.995 61.595) (width 0.5) (layer B.Cu) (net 5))
 (segment (start 87.63 59.055) (end 87.63 60.96) (width 0.5) (layer B.Cu) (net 5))
 (segment (start 88.9 57.785) (end 87.63 59.055) (width 0.5) (layer B.Cu) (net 5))
 (segment (start 92.075 57.785) (end 88.9 57.785) (width 0.5) (layer B.Cu) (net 5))
 (segment (start 93.98 59.69) (end 92.075 57.785) (width 0.5) (layer B.Cu) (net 5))
 (segment (start 83.82 53.34) (end 78.74 53.34) (width 0.5) (layer B.Cu) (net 6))
 (segment (start 78.74 53.34) (end 73.66 58.42) (width 0.5) (layer B.Cu) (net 6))
 (segment (start 60.96 53.34) (end 60.96 54.61) (width 0.5) (layer B.Cu) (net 6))
 (segment (start 60.96 54.61) (end 62.865 56.515) (width 0.5) (layer B.Cu) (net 6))
 (segment (start 62.865 56.515) (end 71.755 56.515) (width 0.5) (layer B.Cu) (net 6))
 (segment (start 71.755 56.515) (end 73.66 58.42) (width 0.5) (layer B.Cu) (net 6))
 (segment (start 85.09 59.69) (end 83.82 58.42) (width 0.5) (layer F.Cu) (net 6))
 (segment (start 83.82 58.42) (end 83.82 53.34) (width 0.5) (layer F.Cu) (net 6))
 (segment (start 90.17 59.69) (end 90.17 60.96) (width 0.5) (layer B.Cu) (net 7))
 (segment (start 77.47 64.135) (end 77.47 69.85) (width 0.5) (layer B.Cu) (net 7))
 (segment (start 78.74 62.865) (end 77.47 64.135) (width 0.5) (layer B.Cu) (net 7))
 (segment (start 88.265 62.865) (end 78.74 62.865) (width 0.5) (layer B.Cu) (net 7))
 (segment (start 90.17 60.96) (end 88.265 62.865) (width 0.5) (layer B.Cu) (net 7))
 (segment (start 80.01 69.85) (end 78.105 69.85) (width 0.5) (layer B.Cu) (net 7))
 (segment (start 78.105 69.85) (end 77.47 69.85) (width 0.5) (layer B.Cu) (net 7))
 (segment (start 77.47 69.85) (end 72.39 69.85) (width 0.5) (layer B.Cu) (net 7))
 (segment (start 72.39 69.85) (end 71.755 69.85) (width 0.5) (layer F.Cu) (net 7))
 (segment (start 71.755 69.85) (end 69.85 67.945) (width 0.5) (layer F.Cu) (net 7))
 (segment (start 69.85 67.945) (end 69.85 60.96) (width 0.5) (layer F.Cu) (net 7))
 (segment (start 69.85 60.96) (end 67.31 58.42) (width 0.5) (layer F.Cu) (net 7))
 (segment (start 80.01 67.31) (end 81.915 67.31) (width 0.5) (layer B.Cu) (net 8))
 (segment (start 92.71 69.85) (end 93.98 68.58) (width 0.5) (layer B.Cu) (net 8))
 (segment (start 84.455 69.85) (end 92.71 69.85) (width 0.5) (layer B.Cu) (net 8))
 (segment (start 81.915 67.31) (end 84.455 69.85) (width 0.5) (layer B.Cu) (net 8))
 (segment (start 80.01 67.31) (end 80.645 67.31) (width 0.5) (layer B.Cu) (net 8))
 (segment (start 72.39 67.31) (end 72.39 64.77) (width 0.5) (layer F.Cu) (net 9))
 (segment (start 52.64 89.38) (end 57.94 89.38) (width 1.5) (layer F.Cu) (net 4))
 (segment (start 59.69 87.63) (end 59.69 80.09) (width 1.5) (layer F.Cu) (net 4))
 (segment (start 57.94 89.38) (end 59.69 87.63) (width 1.5) (layer F.Cu) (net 4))
 (segment (start 57.15 77.55) (end 59.69 80.09) (width 1.5) (layer F.Cu) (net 4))
 (segment (start 59.69 80.09) (end 62.23 77.55) (width 1.5) (layer F.Cu) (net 4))
 (segment (start 62.23 77.55) (end 59.69 75.01) (width 1.5) (layer F.Cu) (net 4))
 (segment (start 59.69 75.01) (end 57.15 77.55) (width 1.5) (layer F.Cu) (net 4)))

